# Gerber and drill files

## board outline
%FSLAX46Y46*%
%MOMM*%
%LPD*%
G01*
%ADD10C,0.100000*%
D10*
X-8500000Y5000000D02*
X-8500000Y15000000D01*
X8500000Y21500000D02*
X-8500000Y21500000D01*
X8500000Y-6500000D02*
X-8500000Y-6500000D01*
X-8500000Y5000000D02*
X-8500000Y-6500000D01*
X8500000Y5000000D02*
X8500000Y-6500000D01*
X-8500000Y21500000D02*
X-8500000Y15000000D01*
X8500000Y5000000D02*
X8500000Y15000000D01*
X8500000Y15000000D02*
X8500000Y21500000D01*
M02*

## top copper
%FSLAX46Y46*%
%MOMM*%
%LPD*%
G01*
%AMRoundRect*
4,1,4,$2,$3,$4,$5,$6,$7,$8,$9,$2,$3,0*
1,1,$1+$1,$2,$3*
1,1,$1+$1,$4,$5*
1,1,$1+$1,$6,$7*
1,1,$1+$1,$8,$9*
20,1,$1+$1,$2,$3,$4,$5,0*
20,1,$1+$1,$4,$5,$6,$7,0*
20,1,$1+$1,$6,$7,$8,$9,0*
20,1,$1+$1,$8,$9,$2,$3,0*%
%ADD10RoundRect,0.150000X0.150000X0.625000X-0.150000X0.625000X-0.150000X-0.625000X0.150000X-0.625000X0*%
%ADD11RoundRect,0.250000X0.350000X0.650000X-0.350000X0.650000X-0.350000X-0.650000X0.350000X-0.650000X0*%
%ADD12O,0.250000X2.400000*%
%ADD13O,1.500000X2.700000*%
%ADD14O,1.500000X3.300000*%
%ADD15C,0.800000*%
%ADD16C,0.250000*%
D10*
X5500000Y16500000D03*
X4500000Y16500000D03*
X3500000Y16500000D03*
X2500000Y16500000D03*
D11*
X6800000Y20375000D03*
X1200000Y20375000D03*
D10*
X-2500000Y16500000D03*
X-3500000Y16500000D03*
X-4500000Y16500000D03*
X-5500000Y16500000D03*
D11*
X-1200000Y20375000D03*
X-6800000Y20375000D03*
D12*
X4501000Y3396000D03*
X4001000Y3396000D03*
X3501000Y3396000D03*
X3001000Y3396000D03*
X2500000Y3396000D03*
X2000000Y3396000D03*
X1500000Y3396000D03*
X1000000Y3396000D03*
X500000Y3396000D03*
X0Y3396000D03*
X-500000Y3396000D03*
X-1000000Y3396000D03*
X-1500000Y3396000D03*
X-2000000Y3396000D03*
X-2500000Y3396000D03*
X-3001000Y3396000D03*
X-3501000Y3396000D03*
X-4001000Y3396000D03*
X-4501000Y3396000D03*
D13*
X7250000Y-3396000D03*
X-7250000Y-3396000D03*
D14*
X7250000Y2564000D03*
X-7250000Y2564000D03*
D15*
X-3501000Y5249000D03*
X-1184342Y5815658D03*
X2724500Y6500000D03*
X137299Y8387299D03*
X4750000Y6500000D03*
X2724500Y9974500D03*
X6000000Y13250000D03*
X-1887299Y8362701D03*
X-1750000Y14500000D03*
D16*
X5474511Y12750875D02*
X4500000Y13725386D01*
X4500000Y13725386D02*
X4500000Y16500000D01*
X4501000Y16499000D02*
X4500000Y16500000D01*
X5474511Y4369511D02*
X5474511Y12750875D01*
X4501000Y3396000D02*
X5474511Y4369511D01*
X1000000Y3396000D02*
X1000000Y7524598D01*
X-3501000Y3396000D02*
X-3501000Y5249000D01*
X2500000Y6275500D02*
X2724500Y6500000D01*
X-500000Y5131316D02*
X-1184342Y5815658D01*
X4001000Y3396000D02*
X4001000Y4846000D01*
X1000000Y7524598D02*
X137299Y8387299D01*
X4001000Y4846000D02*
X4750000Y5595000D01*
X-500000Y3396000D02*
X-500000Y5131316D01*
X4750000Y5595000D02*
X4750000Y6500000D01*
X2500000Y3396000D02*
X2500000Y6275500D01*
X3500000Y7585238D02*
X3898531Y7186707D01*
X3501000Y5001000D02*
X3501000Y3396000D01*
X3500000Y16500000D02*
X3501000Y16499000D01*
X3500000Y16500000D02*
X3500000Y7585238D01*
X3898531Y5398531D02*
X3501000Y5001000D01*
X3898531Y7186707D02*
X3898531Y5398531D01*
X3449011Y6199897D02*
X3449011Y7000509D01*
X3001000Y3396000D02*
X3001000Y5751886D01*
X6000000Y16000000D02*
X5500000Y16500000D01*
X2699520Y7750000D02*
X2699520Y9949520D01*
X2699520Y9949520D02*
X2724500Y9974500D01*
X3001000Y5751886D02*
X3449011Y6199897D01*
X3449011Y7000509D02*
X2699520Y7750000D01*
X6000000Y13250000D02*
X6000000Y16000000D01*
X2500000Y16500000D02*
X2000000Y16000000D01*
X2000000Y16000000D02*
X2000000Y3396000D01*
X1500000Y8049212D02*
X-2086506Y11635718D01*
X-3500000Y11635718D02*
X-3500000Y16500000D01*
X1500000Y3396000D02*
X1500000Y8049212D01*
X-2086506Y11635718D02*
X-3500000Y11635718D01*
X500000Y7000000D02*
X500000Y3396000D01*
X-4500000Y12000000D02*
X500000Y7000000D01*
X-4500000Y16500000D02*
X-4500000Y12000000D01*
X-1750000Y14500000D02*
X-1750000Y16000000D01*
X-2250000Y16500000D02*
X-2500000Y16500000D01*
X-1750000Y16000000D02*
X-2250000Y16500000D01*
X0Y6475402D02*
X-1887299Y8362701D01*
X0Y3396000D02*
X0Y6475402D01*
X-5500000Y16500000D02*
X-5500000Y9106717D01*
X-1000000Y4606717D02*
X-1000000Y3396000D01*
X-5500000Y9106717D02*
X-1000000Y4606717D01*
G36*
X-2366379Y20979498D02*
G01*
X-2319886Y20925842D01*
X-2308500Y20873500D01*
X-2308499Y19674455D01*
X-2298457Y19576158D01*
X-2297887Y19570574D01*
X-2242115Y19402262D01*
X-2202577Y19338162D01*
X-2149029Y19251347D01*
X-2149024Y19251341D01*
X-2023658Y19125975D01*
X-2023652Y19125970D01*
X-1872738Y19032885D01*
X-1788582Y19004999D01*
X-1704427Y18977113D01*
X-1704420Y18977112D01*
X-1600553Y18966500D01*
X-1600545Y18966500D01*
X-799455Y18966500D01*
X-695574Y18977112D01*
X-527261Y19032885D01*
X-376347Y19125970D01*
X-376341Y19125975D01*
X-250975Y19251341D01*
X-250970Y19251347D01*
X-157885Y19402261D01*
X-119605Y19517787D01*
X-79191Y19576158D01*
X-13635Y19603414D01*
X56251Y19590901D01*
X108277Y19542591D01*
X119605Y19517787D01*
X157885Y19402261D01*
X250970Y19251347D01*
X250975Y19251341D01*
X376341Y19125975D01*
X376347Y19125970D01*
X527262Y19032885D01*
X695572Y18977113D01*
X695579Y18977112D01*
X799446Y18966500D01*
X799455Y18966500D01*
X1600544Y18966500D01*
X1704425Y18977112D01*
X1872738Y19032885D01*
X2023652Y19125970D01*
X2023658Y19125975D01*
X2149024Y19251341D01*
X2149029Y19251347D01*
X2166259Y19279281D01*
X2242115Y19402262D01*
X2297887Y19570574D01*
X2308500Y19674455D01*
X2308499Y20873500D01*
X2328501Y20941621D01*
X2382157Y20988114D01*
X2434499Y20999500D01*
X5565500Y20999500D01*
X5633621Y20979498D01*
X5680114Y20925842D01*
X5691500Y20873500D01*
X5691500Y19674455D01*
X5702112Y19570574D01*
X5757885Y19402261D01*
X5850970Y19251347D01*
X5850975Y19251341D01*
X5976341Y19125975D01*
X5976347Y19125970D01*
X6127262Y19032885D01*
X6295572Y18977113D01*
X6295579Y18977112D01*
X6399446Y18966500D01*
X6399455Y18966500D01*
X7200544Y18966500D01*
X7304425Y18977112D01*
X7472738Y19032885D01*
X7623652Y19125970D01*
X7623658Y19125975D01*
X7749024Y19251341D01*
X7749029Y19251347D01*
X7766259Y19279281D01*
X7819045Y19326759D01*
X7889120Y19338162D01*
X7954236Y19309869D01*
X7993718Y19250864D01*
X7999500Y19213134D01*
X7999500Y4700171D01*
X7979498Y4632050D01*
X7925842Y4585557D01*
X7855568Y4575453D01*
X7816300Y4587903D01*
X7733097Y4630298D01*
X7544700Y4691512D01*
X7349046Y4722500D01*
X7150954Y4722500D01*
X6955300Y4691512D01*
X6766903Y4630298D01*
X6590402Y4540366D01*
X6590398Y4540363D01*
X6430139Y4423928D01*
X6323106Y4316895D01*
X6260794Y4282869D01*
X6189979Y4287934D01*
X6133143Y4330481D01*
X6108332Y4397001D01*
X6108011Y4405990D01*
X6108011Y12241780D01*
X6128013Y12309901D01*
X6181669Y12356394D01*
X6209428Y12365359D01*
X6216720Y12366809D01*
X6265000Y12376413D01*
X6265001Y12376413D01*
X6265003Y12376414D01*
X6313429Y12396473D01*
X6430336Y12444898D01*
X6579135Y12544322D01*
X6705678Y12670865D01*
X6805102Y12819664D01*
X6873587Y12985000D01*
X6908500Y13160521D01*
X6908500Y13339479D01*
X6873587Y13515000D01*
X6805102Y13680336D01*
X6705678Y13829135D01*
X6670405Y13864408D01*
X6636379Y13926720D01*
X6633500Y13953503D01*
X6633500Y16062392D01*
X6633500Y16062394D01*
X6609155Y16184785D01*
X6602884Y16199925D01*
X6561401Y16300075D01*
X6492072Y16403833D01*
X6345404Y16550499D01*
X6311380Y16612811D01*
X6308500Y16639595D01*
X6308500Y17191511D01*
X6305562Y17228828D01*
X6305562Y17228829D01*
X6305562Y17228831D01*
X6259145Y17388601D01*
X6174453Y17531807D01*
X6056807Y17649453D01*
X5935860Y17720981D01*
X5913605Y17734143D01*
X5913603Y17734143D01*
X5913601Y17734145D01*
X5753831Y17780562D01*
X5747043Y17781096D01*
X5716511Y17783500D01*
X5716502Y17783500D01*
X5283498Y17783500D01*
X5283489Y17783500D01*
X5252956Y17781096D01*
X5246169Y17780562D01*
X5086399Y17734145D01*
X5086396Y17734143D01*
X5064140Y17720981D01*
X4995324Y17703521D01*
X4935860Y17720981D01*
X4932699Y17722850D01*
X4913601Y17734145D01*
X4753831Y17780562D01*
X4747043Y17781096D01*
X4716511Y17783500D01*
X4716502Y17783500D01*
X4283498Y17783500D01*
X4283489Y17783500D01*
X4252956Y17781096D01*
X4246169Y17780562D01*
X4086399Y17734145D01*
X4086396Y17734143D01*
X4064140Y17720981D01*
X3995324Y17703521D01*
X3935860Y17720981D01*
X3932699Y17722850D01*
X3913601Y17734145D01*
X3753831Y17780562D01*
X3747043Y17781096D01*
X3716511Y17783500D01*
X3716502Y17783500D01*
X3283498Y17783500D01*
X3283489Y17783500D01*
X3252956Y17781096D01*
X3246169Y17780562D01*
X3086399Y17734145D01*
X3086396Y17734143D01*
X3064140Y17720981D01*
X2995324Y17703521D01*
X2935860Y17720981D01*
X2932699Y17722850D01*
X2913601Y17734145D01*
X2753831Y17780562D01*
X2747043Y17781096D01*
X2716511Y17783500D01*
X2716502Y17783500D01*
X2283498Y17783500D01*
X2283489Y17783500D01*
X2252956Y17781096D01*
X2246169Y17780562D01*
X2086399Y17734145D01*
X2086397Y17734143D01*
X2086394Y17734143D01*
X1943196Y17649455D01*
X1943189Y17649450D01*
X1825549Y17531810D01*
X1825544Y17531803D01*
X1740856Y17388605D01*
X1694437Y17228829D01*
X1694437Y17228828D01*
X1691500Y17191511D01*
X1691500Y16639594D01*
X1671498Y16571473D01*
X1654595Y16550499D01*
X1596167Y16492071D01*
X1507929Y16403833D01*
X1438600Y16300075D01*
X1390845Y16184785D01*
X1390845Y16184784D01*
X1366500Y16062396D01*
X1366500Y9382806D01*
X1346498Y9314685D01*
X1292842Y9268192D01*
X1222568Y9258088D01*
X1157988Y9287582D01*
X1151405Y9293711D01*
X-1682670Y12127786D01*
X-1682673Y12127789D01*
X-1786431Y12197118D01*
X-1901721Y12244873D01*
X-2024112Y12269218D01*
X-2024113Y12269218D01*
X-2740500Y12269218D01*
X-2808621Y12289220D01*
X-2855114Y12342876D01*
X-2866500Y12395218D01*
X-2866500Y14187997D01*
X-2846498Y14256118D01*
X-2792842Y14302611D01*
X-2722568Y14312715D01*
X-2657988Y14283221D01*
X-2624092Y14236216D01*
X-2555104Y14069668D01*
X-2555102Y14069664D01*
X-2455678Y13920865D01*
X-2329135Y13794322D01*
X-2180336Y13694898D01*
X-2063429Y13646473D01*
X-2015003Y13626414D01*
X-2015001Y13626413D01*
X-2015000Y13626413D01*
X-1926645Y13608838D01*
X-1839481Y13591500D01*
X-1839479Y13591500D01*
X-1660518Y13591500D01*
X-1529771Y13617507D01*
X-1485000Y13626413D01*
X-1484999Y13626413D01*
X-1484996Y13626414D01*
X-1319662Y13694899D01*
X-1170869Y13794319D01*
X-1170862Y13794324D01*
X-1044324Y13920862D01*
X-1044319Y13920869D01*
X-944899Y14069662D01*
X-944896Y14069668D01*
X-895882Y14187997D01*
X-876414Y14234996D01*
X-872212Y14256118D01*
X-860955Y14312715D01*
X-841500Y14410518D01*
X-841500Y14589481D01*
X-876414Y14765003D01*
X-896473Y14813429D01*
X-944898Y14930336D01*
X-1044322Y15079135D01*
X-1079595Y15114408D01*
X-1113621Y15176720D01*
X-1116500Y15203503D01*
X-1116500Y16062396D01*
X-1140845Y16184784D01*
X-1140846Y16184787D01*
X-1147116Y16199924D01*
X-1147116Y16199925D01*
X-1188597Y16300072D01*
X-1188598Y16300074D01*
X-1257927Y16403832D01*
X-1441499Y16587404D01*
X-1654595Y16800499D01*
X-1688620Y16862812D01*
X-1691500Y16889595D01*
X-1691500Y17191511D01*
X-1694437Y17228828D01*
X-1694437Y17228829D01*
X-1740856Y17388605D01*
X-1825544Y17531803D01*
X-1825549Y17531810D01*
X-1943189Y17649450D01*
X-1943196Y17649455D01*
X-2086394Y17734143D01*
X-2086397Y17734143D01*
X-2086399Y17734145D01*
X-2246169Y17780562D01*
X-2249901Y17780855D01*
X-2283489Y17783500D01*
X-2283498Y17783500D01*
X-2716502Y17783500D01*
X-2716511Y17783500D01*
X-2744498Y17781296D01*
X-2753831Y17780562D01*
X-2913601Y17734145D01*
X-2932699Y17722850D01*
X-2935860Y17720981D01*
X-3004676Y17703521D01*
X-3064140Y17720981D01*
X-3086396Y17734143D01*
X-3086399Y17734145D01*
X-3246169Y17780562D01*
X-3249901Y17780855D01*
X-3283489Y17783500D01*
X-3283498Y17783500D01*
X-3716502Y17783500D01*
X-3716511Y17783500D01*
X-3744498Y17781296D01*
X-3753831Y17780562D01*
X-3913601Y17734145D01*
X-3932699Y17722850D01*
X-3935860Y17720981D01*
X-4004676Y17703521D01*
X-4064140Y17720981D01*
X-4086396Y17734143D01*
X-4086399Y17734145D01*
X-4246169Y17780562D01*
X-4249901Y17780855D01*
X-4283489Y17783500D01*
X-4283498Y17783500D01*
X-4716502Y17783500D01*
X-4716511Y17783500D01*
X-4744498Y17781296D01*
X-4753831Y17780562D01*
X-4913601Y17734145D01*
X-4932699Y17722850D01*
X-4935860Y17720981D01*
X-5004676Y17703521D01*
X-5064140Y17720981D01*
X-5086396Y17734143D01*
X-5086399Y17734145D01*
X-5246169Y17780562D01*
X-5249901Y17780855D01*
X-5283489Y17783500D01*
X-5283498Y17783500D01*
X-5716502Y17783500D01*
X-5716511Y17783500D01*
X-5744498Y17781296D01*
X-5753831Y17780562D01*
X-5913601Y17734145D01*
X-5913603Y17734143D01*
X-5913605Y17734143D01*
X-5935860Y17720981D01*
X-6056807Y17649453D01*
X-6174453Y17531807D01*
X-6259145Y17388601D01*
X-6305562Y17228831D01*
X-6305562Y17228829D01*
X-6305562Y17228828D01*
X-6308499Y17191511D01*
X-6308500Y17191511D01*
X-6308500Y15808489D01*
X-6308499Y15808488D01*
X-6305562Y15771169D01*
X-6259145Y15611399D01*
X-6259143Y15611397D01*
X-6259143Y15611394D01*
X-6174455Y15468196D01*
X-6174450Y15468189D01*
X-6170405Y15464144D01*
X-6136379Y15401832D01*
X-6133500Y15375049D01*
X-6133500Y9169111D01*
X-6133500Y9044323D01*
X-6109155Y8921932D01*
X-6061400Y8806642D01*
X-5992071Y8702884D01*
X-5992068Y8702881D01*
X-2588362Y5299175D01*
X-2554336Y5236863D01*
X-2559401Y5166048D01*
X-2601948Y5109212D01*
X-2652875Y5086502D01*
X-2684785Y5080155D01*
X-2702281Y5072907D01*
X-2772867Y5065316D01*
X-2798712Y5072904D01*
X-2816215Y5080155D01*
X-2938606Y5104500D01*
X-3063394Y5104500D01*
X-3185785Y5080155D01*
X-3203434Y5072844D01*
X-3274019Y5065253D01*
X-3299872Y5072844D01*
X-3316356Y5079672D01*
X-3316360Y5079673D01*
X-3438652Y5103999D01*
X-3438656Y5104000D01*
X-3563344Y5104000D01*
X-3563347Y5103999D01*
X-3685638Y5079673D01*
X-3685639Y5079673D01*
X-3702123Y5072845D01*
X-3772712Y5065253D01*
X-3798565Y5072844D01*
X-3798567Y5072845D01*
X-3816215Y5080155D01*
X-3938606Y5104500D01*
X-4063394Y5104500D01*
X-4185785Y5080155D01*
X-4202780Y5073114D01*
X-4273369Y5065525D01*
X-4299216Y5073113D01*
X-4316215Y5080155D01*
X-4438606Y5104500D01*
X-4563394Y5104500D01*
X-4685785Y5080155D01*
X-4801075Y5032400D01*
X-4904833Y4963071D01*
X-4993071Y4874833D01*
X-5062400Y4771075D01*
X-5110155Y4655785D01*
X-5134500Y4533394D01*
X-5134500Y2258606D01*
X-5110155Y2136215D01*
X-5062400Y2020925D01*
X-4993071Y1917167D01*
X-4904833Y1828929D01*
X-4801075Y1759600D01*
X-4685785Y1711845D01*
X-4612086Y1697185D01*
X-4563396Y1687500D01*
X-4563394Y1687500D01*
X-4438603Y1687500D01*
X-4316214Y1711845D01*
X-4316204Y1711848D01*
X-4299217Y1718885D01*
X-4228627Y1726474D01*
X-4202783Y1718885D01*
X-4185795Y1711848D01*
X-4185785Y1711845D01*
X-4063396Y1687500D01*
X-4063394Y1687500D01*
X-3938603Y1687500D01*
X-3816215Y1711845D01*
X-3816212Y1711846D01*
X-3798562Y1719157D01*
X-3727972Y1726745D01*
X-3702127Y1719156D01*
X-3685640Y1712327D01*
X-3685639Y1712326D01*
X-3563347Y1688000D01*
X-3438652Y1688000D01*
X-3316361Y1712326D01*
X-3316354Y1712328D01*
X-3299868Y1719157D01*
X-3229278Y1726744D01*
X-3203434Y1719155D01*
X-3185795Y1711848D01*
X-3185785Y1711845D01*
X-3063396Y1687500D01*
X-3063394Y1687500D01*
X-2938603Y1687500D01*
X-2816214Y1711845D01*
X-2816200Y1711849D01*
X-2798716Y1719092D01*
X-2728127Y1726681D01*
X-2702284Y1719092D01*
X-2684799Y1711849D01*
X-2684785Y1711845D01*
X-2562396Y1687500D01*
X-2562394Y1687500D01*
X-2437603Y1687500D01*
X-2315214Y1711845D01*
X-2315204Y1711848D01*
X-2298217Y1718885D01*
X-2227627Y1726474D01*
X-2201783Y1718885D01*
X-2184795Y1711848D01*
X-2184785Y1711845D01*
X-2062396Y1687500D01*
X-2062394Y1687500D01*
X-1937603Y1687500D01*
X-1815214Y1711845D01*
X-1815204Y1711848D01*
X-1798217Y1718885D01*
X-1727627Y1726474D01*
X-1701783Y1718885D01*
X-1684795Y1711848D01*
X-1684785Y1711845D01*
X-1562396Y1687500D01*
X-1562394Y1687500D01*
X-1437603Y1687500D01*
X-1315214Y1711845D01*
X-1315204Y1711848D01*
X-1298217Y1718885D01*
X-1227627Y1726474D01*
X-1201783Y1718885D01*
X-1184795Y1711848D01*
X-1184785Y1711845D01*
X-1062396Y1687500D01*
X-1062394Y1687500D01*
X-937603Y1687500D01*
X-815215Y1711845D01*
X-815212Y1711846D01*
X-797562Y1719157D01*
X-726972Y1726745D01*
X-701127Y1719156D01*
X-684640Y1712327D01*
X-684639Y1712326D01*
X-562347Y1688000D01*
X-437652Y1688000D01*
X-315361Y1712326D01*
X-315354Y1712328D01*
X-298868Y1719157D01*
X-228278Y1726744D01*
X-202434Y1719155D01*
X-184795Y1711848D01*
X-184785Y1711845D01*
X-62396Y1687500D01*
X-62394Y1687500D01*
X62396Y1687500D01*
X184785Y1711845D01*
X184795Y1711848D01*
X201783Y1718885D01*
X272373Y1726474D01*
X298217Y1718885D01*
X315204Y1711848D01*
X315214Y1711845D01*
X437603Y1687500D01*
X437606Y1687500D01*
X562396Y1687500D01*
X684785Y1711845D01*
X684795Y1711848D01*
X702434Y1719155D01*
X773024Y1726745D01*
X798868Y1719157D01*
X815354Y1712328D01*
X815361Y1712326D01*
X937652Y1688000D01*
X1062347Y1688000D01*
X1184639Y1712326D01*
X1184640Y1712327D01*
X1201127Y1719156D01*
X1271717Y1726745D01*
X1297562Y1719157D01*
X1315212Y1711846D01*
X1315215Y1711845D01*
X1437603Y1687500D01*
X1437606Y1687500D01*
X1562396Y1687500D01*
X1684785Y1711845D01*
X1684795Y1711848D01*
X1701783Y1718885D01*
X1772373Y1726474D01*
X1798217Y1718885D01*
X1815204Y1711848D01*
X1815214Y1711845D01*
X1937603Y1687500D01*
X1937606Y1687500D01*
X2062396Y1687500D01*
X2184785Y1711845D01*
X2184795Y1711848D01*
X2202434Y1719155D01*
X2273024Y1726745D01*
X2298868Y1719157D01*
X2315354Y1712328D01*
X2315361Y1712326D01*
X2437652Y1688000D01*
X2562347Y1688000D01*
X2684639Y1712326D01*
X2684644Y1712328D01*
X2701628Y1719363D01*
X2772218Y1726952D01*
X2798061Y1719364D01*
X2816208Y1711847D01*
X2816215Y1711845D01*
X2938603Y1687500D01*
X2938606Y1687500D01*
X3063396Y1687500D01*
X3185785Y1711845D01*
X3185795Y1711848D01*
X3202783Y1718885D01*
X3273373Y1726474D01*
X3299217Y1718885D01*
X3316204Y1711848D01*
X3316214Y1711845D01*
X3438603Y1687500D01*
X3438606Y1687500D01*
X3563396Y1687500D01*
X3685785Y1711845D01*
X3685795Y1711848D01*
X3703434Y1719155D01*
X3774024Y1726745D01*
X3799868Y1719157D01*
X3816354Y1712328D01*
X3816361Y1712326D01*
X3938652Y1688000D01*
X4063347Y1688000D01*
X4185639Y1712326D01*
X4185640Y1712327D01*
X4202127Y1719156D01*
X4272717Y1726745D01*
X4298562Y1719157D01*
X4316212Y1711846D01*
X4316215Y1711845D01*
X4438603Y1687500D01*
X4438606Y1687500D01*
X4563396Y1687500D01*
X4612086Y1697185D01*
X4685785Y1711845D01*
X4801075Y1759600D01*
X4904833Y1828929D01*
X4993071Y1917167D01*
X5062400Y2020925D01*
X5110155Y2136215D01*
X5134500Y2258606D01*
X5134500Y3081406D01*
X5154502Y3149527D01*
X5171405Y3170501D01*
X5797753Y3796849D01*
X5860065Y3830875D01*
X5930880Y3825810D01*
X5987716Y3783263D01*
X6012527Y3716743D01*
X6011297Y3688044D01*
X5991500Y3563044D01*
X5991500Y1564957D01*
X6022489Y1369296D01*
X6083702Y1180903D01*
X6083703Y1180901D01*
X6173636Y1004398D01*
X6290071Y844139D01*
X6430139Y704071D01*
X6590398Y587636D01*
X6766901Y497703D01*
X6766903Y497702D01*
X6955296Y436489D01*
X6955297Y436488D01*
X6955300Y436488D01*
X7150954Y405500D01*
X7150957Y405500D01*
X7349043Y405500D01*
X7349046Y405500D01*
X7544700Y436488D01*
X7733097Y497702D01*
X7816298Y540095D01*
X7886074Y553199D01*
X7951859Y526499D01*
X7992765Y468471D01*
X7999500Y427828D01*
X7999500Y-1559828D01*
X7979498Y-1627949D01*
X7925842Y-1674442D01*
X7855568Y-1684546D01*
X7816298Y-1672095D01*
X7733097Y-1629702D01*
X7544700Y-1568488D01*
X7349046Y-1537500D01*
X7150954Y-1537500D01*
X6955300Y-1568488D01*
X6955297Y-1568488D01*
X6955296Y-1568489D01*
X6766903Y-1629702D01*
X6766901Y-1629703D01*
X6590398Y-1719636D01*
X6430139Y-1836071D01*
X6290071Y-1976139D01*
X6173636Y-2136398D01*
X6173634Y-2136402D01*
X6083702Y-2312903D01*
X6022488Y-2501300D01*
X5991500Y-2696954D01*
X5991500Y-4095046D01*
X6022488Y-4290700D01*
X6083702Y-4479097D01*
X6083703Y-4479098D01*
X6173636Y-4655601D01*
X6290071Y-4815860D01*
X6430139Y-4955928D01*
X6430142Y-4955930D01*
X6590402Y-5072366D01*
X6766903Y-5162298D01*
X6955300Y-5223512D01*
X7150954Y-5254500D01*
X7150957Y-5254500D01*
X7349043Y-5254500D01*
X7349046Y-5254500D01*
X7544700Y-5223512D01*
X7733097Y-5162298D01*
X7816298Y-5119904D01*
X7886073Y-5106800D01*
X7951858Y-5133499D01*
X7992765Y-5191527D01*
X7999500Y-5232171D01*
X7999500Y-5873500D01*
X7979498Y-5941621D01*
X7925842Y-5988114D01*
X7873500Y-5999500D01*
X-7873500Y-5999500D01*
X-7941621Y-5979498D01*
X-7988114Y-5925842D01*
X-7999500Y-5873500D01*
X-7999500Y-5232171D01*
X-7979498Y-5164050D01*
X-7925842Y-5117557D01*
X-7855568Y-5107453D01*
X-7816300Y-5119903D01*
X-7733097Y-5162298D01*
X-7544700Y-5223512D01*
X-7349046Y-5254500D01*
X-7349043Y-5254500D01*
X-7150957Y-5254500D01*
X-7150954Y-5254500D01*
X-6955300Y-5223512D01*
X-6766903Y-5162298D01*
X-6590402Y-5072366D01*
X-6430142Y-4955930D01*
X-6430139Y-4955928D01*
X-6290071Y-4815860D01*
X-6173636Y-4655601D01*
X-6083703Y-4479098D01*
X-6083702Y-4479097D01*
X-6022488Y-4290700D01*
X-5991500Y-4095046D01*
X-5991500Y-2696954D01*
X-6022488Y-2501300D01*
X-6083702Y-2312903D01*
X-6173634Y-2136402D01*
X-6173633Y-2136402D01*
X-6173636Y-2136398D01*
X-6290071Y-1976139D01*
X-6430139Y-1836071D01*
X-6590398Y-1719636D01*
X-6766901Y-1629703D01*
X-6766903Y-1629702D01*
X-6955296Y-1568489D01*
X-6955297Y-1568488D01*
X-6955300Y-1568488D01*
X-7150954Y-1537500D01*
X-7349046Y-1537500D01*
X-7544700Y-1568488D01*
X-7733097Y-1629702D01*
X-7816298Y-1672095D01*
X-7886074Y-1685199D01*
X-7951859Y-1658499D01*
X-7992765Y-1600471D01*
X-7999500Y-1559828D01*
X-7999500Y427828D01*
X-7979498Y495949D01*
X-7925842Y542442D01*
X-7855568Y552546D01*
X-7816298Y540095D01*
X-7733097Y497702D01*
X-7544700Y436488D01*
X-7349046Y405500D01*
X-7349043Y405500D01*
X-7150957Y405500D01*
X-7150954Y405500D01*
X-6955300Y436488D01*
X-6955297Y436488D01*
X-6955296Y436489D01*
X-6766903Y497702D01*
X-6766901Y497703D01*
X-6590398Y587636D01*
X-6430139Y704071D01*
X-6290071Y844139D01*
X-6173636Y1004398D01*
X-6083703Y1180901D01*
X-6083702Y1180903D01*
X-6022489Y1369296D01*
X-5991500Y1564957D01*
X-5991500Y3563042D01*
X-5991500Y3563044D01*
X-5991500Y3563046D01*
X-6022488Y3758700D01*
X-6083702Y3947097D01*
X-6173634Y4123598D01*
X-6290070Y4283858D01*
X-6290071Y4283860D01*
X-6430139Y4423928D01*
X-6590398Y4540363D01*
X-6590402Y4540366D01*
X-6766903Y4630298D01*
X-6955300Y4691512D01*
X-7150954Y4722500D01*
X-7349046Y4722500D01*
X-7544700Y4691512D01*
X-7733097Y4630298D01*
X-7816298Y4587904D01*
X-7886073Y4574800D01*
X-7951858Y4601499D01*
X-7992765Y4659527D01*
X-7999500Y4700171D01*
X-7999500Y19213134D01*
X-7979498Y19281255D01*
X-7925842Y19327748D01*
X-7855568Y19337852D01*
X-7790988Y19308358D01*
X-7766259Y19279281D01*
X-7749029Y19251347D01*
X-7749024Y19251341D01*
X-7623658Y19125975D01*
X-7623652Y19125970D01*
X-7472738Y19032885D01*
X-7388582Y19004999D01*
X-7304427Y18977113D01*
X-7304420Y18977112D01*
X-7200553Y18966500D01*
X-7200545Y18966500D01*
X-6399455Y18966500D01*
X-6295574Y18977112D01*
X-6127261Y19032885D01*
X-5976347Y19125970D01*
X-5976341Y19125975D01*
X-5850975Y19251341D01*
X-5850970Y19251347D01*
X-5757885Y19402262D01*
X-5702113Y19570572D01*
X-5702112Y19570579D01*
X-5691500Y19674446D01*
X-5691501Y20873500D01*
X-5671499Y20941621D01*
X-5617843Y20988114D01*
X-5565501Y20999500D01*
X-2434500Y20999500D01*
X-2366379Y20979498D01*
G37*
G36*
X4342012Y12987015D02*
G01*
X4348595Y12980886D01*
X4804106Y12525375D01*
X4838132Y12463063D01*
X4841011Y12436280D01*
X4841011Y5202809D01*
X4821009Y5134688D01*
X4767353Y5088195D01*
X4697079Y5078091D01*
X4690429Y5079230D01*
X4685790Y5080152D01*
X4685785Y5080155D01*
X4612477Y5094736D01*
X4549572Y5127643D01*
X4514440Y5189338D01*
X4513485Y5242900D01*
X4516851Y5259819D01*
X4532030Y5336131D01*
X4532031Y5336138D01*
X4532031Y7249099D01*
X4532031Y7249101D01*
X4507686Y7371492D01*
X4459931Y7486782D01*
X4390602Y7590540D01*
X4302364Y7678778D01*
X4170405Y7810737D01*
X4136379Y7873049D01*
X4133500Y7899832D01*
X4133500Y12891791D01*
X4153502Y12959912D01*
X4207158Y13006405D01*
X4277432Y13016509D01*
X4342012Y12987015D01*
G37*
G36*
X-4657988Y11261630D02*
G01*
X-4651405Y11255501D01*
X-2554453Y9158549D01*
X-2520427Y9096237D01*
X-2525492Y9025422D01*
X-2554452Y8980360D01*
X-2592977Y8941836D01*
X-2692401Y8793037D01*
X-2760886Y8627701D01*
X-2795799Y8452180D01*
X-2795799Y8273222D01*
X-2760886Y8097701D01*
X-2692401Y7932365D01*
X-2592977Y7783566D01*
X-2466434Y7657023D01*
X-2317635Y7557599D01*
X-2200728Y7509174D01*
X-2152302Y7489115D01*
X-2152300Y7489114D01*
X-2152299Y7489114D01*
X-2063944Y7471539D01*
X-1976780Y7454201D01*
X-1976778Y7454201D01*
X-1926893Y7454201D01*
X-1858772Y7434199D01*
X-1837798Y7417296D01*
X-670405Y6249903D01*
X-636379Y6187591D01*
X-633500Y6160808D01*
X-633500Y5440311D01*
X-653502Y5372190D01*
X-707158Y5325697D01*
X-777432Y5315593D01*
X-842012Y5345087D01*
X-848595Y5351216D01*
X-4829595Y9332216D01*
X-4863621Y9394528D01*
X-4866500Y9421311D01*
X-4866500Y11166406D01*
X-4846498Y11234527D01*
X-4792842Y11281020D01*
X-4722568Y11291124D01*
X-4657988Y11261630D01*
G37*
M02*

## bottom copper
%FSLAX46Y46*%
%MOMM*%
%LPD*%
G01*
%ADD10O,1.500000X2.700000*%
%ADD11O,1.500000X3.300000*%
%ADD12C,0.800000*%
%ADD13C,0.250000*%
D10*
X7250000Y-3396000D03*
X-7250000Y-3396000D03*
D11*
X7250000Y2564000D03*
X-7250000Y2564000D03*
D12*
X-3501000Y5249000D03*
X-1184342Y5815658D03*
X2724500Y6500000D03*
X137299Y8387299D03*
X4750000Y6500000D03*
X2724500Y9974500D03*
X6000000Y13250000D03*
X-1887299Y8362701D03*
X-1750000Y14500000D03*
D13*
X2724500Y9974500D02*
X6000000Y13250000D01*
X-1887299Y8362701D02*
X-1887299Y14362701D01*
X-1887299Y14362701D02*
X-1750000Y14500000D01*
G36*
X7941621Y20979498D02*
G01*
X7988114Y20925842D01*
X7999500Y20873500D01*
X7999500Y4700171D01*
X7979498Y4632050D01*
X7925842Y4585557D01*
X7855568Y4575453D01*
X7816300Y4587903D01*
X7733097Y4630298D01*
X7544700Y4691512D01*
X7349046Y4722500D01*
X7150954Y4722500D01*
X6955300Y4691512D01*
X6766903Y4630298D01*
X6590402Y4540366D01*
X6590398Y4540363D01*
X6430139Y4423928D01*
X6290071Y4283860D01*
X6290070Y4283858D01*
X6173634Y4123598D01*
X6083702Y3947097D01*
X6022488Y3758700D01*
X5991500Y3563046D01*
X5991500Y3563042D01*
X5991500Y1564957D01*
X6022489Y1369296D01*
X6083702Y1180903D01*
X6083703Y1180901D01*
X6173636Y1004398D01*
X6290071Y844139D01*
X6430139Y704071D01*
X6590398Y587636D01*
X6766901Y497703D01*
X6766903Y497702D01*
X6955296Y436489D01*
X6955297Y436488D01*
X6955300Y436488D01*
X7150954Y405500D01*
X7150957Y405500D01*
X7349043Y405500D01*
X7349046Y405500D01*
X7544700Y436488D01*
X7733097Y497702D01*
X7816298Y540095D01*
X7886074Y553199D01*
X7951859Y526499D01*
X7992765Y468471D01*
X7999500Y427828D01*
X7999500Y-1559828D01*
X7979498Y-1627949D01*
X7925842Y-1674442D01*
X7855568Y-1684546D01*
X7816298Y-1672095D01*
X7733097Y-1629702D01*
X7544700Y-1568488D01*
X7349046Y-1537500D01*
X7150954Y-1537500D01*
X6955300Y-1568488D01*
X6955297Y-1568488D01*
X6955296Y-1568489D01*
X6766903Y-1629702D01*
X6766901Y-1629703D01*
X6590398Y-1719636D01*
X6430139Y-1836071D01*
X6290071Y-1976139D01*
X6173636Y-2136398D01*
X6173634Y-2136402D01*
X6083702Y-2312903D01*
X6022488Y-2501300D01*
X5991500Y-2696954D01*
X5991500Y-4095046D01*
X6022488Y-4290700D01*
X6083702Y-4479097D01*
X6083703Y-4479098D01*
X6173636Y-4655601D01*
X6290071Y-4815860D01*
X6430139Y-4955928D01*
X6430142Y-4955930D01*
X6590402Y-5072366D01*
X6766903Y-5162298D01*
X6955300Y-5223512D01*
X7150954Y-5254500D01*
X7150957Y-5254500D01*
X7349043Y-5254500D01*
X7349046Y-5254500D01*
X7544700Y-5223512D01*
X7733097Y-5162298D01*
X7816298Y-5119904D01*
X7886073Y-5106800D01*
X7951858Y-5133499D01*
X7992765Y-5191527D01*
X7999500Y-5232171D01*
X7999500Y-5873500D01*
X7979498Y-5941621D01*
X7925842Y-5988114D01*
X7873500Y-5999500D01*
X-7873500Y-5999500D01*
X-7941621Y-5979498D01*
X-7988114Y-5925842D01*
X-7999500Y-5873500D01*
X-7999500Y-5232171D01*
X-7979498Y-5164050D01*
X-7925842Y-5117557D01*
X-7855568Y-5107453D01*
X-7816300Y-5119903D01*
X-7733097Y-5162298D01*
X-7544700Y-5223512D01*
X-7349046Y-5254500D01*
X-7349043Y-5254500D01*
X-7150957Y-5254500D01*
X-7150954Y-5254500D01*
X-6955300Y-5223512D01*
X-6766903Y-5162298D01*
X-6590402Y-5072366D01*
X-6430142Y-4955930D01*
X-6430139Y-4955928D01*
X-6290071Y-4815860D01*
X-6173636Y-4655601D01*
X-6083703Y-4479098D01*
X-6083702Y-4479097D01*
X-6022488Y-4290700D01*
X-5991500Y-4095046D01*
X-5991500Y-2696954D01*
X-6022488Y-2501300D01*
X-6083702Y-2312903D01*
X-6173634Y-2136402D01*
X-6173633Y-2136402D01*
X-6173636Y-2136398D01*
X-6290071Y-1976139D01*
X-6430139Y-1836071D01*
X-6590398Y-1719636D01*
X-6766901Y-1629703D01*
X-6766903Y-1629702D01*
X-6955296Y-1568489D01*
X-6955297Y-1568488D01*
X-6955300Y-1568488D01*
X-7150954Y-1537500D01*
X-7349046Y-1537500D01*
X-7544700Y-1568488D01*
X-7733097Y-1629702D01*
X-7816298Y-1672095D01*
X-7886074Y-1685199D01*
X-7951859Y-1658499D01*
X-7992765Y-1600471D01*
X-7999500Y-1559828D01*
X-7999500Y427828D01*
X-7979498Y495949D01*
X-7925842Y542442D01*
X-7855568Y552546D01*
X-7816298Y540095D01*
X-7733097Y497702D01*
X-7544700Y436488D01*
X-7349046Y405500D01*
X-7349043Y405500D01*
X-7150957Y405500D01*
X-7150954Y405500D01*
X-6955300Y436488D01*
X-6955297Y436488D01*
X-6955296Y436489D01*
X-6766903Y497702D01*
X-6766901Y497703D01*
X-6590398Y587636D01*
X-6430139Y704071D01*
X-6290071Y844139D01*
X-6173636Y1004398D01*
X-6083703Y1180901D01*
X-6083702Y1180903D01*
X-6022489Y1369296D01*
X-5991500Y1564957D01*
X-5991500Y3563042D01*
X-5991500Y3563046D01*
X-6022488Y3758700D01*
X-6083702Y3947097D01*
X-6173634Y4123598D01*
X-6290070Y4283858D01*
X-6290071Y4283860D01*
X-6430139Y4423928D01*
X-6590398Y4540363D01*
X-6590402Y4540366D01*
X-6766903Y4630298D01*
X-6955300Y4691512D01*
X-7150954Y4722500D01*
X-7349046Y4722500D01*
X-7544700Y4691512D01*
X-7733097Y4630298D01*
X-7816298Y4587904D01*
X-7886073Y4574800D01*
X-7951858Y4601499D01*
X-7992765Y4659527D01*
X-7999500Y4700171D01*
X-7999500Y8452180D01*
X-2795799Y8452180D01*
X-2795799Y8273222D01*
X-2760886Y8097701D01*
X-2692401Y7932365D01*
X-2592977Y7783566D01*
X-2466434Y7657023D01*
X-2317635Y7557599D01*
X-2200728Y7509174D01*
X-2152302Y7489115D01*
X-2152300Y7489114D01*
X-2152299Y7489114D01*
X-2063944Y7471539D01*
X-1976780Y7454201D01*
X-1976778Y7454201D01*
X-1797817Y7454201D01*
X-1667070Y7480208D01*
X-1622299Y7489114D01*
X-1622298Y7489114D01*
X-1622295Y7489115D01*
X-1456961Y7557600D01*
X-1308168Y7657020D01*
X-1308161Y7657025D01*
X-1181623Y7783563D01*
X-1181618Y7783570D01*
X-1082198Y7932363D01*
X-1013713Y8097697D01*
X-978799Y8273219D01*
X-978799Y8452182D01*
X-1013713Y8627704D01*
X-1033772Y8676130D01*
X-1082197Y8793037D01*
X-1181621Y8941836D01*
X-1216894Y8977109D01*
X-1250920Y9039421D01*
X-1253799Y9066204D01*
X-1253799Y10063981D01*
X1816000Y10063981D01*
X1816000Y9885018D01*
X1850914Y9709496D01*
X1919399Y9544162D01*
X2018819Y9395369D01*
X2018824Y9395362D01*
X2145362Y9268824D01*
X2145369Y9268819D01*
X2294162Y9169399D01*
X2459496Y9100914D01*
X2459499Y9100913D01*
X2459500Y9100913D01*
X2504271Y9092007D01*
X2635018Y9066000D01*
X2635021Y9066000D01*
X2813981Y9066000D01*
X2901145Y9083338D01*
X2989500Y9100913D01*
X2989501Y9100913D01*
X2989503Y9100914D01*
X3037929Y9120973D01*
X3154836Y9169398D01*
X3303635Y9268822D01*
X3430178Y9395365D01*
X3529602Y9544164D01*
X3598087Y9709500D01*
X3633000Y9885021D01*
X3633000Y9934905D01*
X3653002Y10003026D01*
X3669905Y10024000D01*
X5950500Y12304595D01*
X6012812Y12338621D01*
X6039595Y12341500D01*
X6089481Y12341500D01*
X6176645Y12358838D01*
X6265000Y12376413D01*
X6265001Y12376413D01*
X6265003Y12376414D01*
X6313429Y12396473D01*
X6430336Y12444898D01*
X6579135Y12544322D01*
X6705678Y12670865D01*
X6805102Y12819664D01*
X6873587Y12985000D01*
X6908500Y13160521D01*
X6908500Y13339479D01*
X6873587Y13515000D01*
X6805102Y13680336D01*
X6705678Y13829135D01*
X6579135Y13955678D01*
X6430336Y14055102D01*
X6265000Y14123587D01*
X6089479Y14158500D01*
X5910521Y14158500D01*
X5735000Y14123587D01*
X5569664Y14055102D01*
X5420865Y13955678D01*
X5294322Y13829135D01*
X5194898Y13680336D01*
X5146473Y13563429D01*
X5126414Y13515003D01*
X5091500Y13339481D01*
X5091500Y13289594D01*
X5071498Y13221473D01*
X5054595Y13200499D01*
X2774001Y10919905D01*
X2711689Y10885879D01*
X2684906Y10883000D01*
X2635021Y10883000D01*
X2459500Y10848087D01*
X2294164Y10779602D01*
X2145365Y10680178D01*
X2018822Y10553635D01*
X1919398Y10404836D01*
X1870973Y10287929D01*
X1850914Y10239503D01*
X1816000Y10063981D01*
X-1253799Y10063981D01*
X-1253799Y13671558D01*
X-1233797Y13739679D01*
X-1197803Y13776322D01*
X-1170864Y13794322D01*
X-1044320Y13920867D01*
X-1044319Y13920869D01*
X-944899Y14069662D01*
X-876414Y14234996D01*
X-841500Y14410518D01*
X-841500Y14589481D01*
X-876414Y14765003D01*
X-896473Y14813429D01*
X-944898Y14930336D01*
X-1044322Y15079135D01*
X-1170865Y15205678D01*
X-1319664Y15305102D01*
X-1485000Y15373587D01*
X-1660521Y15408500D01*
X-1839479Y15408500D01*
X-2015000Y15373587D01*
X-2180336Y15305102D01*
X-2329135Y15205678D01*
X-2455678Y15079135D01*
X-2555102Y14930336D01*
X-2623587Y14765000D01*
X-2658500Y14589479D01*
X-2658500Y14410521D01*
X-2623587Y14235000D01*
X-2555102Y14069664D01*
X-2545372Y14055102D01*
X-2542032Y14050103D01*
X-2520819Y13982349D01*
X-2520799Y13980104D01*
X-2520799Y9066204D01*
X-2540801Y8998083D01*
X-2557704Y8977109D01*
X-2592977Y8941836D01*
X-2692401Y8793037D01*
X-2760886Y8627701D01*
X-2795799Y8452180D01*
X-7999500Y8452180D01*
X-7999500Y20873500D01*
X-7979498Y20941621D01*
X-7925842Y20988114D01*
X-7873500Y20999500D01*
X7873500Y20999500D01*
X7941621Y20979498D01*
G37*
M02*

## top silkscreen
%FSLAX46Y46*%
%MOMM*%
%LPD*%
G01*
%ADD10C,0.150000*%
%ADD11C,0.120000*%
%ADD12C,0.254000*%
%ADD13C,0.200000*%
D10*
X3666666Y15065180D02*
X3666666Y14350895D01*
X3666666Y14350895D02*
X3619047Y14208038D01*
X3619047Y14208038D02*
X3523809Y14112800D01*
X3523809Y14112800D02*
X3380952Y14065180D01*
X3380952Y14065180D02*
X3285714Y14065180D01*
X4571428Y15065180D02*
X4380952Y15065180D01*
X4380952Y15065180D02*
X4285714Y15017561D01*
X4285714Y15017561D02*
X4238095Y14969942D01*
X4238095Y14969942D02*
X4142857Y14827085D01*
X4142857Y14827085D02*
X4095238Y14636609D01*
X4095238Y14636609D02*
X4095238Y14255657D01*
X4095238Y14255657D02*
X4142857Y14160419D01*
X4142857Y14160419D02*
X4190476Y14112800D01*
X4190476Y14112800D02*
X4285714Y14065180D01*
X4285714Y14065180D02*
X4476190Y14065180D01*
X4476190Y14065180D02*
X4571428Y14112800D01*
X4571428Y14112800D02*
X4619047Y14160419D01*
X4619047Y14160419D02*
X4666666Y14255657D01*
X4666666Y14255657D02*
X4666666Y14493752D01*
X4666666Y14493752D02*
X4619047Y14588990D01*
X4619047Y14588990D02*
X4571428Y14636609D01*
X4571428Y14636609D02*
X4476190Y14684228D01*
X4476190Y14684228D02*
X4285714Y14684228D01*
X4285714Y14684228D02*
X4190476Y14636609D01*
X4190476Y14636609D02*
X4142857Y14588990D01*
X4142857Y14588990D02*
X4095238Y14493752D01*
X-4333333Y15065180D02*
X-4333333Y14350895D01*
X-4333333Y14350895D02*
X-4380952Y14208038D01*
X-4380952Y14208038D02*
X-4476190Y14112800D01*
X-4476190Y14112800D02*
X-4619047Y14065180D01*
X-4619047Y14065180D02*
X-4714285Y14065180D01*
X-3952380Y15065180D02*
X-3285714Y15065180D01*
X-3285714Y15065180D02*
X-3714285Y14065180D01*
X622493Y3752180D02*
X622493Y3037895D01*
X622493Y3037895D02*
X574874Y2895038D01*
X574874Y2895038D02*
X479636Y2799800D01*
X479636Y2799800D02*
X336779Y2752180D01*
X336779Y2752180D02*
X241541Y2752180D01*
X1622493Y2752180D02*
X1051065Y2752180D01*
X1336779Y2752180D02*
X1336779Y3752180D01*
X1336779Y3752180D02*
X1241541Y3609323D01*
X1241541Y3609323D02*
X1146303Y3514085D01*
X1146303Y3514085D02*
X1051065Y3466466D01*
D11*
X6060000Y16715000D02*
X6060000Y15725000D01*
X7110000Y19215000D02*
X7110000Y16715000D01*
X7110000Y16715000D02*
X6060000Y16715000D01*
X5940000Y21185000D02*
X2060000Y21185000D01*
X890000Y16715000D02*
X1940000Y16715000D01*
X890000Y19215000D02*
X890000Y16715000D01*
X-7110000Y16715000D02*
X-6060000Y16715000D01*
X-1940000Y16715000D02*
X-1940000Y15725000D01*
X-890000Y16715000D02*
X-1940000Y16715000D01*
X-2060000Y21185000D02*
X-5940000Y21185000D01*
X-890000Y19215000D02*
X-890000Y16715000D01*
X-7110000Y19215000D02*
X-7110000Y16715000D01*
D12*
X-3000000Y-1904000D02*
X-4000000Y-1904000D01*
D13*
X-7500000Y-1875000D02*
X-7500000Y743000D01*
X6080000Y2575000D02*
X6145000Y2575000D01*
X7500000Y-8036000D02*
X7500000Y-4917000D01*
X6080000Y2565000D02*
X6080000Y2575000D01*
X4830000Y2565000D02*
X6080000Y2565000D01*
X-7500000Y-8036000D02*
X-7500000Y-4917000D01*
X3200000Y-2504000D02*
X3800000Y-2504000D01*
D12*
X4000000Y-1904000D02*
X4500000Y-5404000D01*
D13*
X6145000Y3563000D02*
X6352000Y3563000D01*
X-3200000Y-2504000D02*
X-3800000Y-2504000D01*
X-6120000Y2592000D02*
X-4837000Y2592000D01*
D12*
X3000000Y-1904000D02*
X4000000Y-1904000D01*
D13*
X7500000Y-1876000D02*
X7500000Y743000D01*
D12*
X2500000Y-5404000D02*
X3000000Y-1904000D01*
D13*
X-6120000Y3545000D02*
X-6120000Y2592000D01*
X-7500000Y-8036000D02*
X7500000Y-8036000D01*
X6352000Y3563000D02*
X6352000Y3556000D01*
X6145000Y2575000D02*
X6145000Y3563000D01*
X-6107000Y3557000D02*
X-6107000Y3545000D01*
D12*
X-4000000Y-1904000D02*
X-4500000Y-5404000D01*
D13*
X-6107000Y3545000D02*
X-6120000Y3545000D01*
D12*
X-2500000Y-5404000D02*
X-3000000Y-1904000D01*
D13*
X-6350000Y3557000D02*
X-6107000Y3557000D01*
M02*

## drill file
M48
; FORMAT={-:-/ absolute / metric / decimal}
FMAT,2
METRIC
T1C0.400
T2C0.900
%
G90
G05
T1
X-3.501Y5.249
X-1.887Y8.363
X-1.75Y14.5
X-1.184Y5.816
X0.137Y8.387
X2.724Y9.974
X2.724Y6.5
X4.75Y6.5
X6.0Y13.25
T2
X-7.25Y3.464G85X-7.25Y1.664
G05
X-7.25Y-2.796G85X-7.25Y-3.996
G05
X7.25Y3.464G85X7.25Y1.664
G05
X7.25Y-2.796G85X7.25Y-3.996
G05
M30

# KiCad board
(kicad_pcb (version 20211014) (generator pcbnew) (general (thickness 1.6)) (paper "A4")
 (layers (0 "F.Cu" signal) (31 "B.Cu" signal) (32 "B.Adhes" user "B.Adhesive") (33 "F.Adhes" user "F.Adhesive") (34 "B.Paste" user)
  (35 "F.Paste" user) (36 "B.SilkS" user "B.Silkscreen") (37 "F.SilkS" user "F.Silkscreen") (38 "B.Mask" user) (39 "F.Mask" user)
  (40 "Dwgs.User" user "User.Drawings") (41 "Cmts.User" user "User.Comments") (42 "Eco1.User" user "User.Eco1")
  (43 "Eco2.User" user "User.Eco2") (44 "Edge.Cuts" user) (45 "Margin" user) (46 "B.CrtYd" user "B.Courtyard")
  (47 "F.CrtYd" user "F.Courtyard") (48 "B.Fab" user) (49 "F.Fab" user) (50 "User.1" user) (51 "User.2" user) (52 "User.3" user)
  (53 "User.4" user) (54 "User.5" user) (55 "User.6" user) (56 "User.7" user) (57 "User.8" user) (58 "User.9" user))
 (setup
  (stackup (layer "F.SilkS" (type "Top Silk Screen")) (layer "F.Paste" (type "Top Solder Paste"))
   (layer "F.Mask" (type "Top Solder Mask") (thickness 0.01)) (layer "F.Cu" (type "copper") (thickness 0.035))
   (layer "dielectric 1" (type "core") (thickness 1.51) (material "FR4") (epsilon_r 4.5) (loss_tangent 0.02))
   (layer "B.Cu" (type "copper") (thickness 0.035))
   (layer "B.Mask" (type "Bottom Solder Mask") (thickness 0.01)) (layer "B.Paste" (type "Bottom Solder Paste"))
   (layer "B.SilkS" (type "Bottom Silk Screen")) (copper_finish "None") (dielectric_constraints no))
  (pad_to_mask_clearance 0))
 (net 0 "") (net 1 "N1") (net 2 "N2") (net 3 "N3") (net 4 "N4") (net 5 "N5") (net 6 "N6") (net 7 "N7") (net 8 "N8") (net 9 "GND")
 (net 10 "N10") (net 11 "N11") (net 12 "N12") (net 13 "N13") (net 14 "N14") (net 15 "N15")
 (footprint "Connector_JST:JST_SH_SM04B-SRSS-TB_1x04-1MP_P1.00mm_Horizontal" (layer "F.Cu") (at 4 -18.5 180)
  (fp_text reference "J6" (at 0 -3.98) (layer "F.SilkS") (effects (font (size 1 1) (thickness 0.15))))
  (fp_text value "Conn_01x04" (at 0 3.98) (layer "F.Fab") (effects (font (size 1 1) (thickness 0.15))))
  (fp_line (start -2.06 -1.785) (end -2.06 -2.775) (layer "F.SilkS") (width 0.12))
  (fp_line (start -3.11 0.715) (end -3.11 -1.785) (layer "F.SilkS") (width 0.12))
  (fp_line (start -3.11 -1.785) (end -2.06 -1.785) (layer "F.SilkS") (width 0.12))
  (fp_line (start -1.94 2.685) (end 1.94 2.685) (layer "F.SilkS") (width 0.12))
  (fp_line (start 3.11 -1.785) (end 2.06 -1.785) (layer "F.SilkS") (width 0.12))
  (fp_line (start 3.11 0.715) (end 3.11 -1.785) (layer "F.SilkS") (width 0.12))
  (pad "1" smd roundrect (at -1.5 -2 180) (size 0.6 1.55) (layers "F.Cu" "F.Paste" "F.Mask") (roundrect_rratio 0.25) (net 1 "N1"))
  (pad "2" smd roundrect (at -0.5 -2 180) (size 0.6 1.55) (layers "F.Cu" "F.Paste" "F.Mask") (roundrect_rratio 0.25) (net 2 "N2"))
  (pad "3" smd roundrect (at 0.5 -2 180) (size 0.6 1.55) (layers "F.Cu" "F.Paste" "F.Mask") (roundrect_rratio 0.25) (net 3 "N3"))
  (pad "4" smd roundrect (at 1.5 -2 180) (size 0.6 1.55) (layers "F.Cu" "F.Paste" "F.Mask") (roundrect_rratio 0.25) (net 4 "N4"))
  (pad "MP" smd roundrect (at -2.8 1.875 180) (size 1.2 1.8) (layers "F.Cu" "F.Paste" "F.Mask") (roundrect_rratio 0.2083333333))
  (pad "MP" smd roundrect (at 2.8 1.875 180) (size 1.2 1.8) (layers "F.Cu" "F.Paste" "F.Mask") (roundrect_rratio 0.2083333333)))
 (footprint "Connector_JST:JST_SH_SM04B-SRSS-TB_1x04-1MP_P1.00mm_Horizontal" (layer "F.Cu") (at -4 -18.5 180)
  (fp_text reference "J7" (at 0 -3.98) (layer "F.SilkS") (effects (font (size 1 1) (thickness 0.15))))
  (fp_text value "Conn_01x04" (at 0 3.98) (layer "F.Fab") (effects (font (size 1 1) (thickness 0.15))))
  (fp_line (start 3.11 -1.785) (end 2.06 -1.785) (layer "F.SilkS") (width 0.12))
  (fp_line (start -2.06 -1.785) (end -2.06 -2.775) (layer "F.SilkS") (width 0.12))
  (fp_line (start -3.11 -1.785) (end -2.06 -1.785) (layer "F.SilkS") (width 0.12))
  (fp_line (start -1.94 2.685) (end 1.94 2.685) (layer "F.SilkS") (width 0.12))
  (fp_line (start -3.11 0.715) (end -3.11 -1.785) (layer "F.SilkS") (width 0.12))
  (fp_line (start 3.11 0.715) (end 3.11 -1.785) (layer "F.SilkS") (width 0.12))
  (pad "1" smd roundrect (at -1.5 -2 180) (size 0.6 1.55) (layers "F.Cu" "F.Paste" "F.Mask") (roundrect_rratio 0.25) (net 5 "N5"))
  (pad "2" smd roundrect (at -0.5 -2 180) (size 0.6 1.55) (layers "F.Cu" "F.Paste" "F.Mask") (roundrect_rratio 0.25) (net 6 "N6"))
  (pad "3" smd roundrect (at 0.5 -2 180) (size 0.6 1.55) (layers "F.Cu" "F.Paste" "F.Mask") (roundrect_rratio 0.25) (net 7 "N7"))
  (pad "4" smd roundrect (at 1.5 -2 180) (size 0.6 1.55) (layers "F.Cu" "F.Paste" "F.Mask") (roundrect_rratio 0.25) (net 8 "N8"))
  (pad "MP" smd roundrect (at -2.8 1.875 180) (size 1.2 1.8) (layers "F.Cu" "F.Paste" "F.Mask") (roundrect_rratio 0.2083333333))
  (pad "MP" smd roundrect (at 2.8 1.875 180) (size 1.2 1.8) (layers "F.Cu" "F.Paste" "F.Mask") (roundrect_rratio 0.2083333333)))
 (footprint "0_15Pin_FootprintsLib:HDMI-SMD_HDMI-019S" (layer "F.Cu") (at 0 0)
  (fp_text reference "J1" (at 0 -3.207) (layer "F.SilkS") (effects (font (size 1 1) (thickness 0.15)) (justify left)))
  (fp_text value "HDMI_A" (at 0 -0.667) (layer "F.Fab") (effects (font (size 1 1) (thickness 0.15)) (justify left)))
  (fp_line (start -3 1.904) (end -4 1.904) (layer "F.SilkS") (width 0.254))
  (fp_line (start -7.5 1.875) (end -7.5 -0.743) (layer "F.SilkS") (width 0.2))
  (fp_line (start 6.08 -2.575) (end 6.145 -2.575) (layer "F.SilkS") (width 0.2))
  (fp_line (start 7.5 8.036) (end 7.5 4.917) (layer "F.SilkS") (width 0.2))
  (fp_line (start 6.08 -2.565) (end 6.08 -2.575) (layer "F.SilkS") (width 0.2))
  (fp_line (start 4.83 -2.565) (end 6.08 -2.565) (layer "F.SilkS") (width 0.2))
  (fp_line (start -7.5 8.036) (end -7.5 4.917) (layer "F.SilkS") (width 0.2))
  (fp_line (start 3.2 2.504) (end 3.8 2.504) (layer "F.SilkS") (width 0.2))
  (fp_line (start 4 1.904) (end 4.5 5.404) (layer "F.SilkS") (width 0.254))
  (fp_line (start 6.145 -3.563) (end 6.352 -3.563) (layer "F.SilkS") (width 0.2))
  (fp_line (start -3.2 2.504) (end -3.8 2.504) (layer "F.SilkS") (width 0.2))
  (fp_line (start -6.12 -2.592) (end -4.837 -2.592) (layer "F.SilkS") (width 0.2))
  (fp_line (start 3 1.904) (end 4 1.904) (layer "F.SilkS") (width 0.254))
  (fp_line (start 7.5 1.876) (end 7.5 -0.743) (layer "F.SilkS") (width 0.2))
  (fp_line (start 2.5 5.404) (end 3 1.904) (layer "F.SilkS") (width 0.254))
  (fp_line (start -6.12 -3.545) (end -6.12 -2.592) (layer "F.SilkS") (width 0.2))
  (fp_line (start -7.5 8.036) (end 7.5 8.036) (layer "F.SilkS") (width 0.2))
  (fp_line (start 6.352 -3.563) (end 6.352 -3.556) (layer "F.SilkS") (width 0.2))
  (fp_line (start 6.145 -2.575) (end 6.145 -3.563) (layer "F.SilkS") (width 0.2))
  (fp_line (start -6.107 -3.557) (end -6.107 -3.545) (layer "F.SilkS") (width 0.2))
  (fp_line (start -4 1.904) (end -4.5 5.404) (layer "F.SilkS") (width 0.254))
  (fp_line (start -6.107 -3.545) (end -6.12 -3.545) (layer "F.SilkS") (width 0.2))
  (fp_line (start -2.5 5.404) (end -3 1.904) (layer "F.SilkS") (width 0.254))
  (fp_line (start -6.35 -3.557) (end -6.107 -3.557) (layer "F.SilkS") (width 0.2))
  (pad "1" smd oval (at 4.501 -3.396) (size 0.25 2.4) (layers "F.Cu" "F.Paste" "F.Mask") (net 2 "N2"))
  (pad "2" smd oval (at 4.001 -3.396) (size 0.25 2.4) (layers "F.Cu" "F.Paste" "F.Mask") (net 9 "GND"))
  (pad "3" smd oval (at 3.501 -3.396) (size 0.25 2.4) (layers "F.Cu" "F.Paste" "F.Mask") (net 3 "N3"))
  (pad "4" smd oval (at 3.001 -3.396) (size 0.25 2.4) (layers "F.Cu" "F.Paste" "F.Mask") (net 1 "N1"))
  (pad "5" smd oval (at 2.5 -3.396) (size 0.25 2.4) (layers "F.Cu" "F.Paste" "F.Mask") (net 9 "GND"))
  (pad "6" smd oval (at 2 -3.396) (size 0.25 2.4) (layers "F.Cu" "F.Paste" "F.Mask") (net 4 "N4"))
  (pad "7" smd oval (at 1.5 -3.396) (size 0.25 2.4) (layers "F.Cu" "F.Paste" "F.Mask") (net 6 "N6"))
  (pad "8" smd oval (at 1 -3.396) (size 0.25 2.4) (layers "F.Cu" "F.Paste" "F.Mask") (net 9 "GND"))
  (pad "9" smd oval (at 0.5 -3.396) (size 0.25 2.4) (layers "F.Cu" "F.Paste" "F.Mask") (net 7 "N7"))
  (pad "10" smd oval (at 0 -3.396) (size 0.25 2.4) (layers "F.Cu" "F.Paste" "F.Mask") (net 5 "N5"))
  (pad "11" smd oval (at -0.5 -3.396) (size 0.25 2.4) (layers "F.Cu" "F.Paste" "F.Mask") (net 9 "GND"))
  (pad "12" smd oval (at -1 -3.396) (size 0.25 2.4) (layers "F.Cu" "F.Paste" "F.Mask") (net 8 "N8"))
  (pad "13" smd oval (at -1.5 -3.396) (size 0.25 2.4) (layers "F.Cu" "F.Paste" "F.Mask") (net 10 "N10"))
  (pad "14" smd oval (at -2 -3.396) (size 0.25 2.4) (layers "F.Cu" "F.Paste" "F.Mask") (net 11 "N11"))
  (pad "15" smd oval (at -2.5 -3.396) (size 0.25 2.4) (layers "F.Cu" "F.Paste" "F.Mask") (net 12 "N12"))
  (pad "16" smd oval (at -3.001 -3.396) (size 0.25 2.4) (layers "F.Cu" "F.Paste" "F.Mask") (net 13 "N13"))
  (pad "17" smd oval (at -3.501 -3.396) (size 0.25 2.4) (layers "F.Cu" "F.Paste" "F.Mask") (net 9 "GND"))
  (pad "18" smd oval (at -4.001 -3.396) (size 0.25 2.4) (layers "F.Cu" "F.Paste" "F.Mask") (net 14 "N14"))
  (pad "19" smd oval (at -4.501 -3.396) (size 0.25 2.4) (layers "F.Cu" "F.Paste" "F.Mask") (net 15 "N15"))
  (pad "20" thru_hole oval (at 7.25 3.396) (size 1.5 2.7) (drill oval 0.9 2.1) (layers *.Cu *.Mask))
  (pad "21" thru_hole oval (at -7.25 3.396) (size 1.5 2.7) (drill oval 0.9 2.1) (layers *.Cu *.Mask))
  (pad "22" thru_hole oval (at 7.25 -2.564) (size 1.5 3.3) (drill oval 0.9 2.7) (layers *.Cu *.Mask))
  (pad "23" thru_hole oval (at -7.25 -2.564) (size 1.5 3.3) (drill oval 0.9 2.7) (layers *.Cu *.Mask)))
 (gr_line (start -8.5 -5) (end -8.5 -15) (layer "Edge.Cuts") (width 0.1))
 (gr_line (start 8.5 -21.5) (end -8.5 -21.5) (layer "Edge.Cuts") (width 0.1))
 (gr_line (start 8.5 6.5) (end -8.5 6.5) (layer "Edge.Cuts") (width 0.1))
 (gr_line (start -8.5 -5) (end -8.5 6.5) (layer "Edge.Cuts") (width 0.1))
 (gr_line (start 8.5 -5) (end 8.5 6.5) (layer "Edge.Cuts") (width 0.1))
 (gr_line (start -8.5 -21.5) (end -8.5 -15) (layer "Edge.Cuts") (width 0.1))
 (gr_line (start 8.5 -5) (end 8.5 -15) (layer "Edge.Cuts") (width 0.1))
 (gr_line (start 8.5 -15) (end 8.5 -21.5) (layer "Edge.Cuts") (width 0.1))
 (segment (start 5.474511 -12.750875) (end 4.5 -13.725386) (width 0.25) (layer "F.Cu") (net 2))
 (segment (start 4.5 -13.725386) (end 4.5 -16.5) (width 0.25) (layer "F.Cu") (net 2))
 (segment (start 4.501 -16.499) (end 4.5 -16.5) (width 0.25) (layer "F.Cu") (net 2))
 (segment (start 5.474511 -4.369511) (end 5.474511 -12.750875) (width 0.25) (layer "F.Cu") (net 2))
 (segment (start 4.501 -3.396) (end 5.474511 -4.369511) (width 0.25) (layer "F.Cu") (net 2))
 (segment (start 1 -3.396) (end 1 -7.524598) (width 0.25) (layer "F.Cu") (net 9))
 (segment (start -3.501 -3.396) (end -3.501 -5.249) (width 0.25) (layer "F.Cu") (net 9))
 (segment (start 2.5 -6.2755) (end 2.7245 -6.5) (width 0.25) (layer "F.Cu") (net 9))
 (segment (start -0.5 -5.131316) (end -1.184342 -5.815658) (width 0.25) (layer "F.Cu") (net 9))
 (segment (start 4.001 -3.396) (end 4.001 -4.846) (width 0.25) (layer "F.Cu") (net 9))
 (segment (start 1 -7.524598) (end 0.137299 -8.387299) (width 0.25) (layer "F.Cu") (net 9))
 (segment (start 4.001 -4.846) (end 4.75 -5.595) (width 0.25) (layer "F.Cu") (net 9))
 (segment (start -0.5 -3.396) (end -0.5 -5.131316) (width 0.25) (layer "F.Cu") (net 9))
 (segment (start 4.75 -5.595) (end 4.75 -6.5) (width 0.25) (layer "F.Cu") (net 9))
 (segment (start 2.5 -3.396) (end 2.5 -6.2755) (width 0.25) (layer "F.Cu") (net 9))
 (via (at -3.501 -5.249) (size 0.8) (drill 0.4) (layers "F.Cu" "B.Cu") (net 9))
 (via (at -1.184342 -5.815658) (size 0.8) (drill 0.4) (layers "F.Cu" "B.Cu") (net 9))
 (via (at 2.7245 -6.5) (size 0.8) (drill 0.4) (layers "F.Cu" "B.Cu") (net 9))
 (via (at 0.137299 -8.387299) (size 0.8) (drill 0.4) (layers "F.Cu" "B.Cu") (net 9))
 (via (at 4.75 -6.5) (size 0.8) (drill 0.4) (layers "F.Cu" "B.Cu") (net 9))
 (segment (start 3.5 -7.585238) (end 3.898531 -7.186707) (width 0.25) (layer "F.Cu") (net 3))
 (segment (start 3.501 -5.001) (end 3.501 -3.396) (width 0.25) (layer "F.Cu") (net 3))
 (segment (start 3.5 -16.5) (end 3.501 -16.499) (width 0.25) (layer "F.Cu") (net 3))
 (segment (start 3.5 -16.5) (end 3.5 -7.585238) (width 0.25) (layer "F.Cu") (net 3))
 (segment (start 3.898531 -5.398531) (end 3.501 -5.001) (width 0.25) (layer "F.Cu") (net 3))
 (segment (start 3.898531 -7.186707) (end 3.898531 -5.398531) (width 0.25) (layer "F.Cu") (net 3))
 (segment (start 3.449011 -6.199897) (end 3.449011 -7.000509) (width 0.25) (layer "F.Cu") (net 1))
 (segment (start 3.001 -3.396) (end 3.001 -5.751886) (width 0.25) (layer "F.Cu") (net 1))
 (segment (start 6 -16) (end 5.5 -16.5) (width 0.25) (layer "F.Cu") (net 1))
 (segment (start 2.69952 -7.75) (end 2.69952 -9.94952) (width 0.25) (layer "F.Cu") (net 1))
 (segment (start 2.69952 -9.94952) (end 2.7245 -9.9745) (width 0.25) (layer "F.Cu") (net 1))
 (segment (start 3.001 -5.751886) (end 3.449011 -6.199897) (width 0.25) (layer "F.Cu") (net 1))
 (segment (start 3.449011 -7.000509) (end 2.69952 -7.75) (width 0.25) (layer "F.Cu") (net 1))
 (segment (start 6 -13.25) (end 6 -16) (width 0.25) (layer "F.Cu") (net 1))
 (via (at 2.7245 -9.9745) (size 0.8) (drill 0.4) (layers "F.Cu" "B.Cu") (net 1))
 (via (at 6 -13.25) (size 0.8) (drill 0.4) (layers "F.Cu" "B.Cu") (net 1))
 (segment (start 2.7245 -9.9745) (end 6 -13.25) (width 0.25) (layer "B.Cu") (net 1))
 (segment (start 2.5 -16.5) (end 2 -16) (width 0.25) (layer "F.Cu") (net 4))
 (segment (start 2 -16) (end 2 -3.396) (width 0.25) (layer "F.Cu") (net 4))
 (segment (start 1.5 -8.049212) (end -2.086506 -11.635718) (width 0.25) (layer "F.Cu") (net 6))
 (segment (start -3.5 -11.635718) (end -3.5 -16.5) (width 0.25) (layer "F.Cu") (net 6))
 (segment (start 1.5 -3.396) (end 1.5 -8.049212) (width 0.25) (layer "F.Cu") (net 6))
 (segment (start -2.086506 -11.635718) (end -3.5 -11.635718) (width 0.25) (layer "F.Cu") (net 6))
 (segment (start 0.5 -7) (end 0.5 -3.396) (width 0.25) (layer "F.Cu") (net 7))
 (segment (start -4.5 -12) (end 0.5 -7) (width 0.25) (layer "F.Cu") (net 7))
 (segment (start -4.5 -16.5) (end -4.5 -12) (width 0.25) (layer "F.Cu") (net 7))
 (segment (start -1.75 -14.5) (end -1.75 -16) (width 0.25) (layer "F.Cu") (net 5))
 (segment (start -2.25 -16.5) (end -2.5 -16.5) (width 0.25) (layer "F.Cu") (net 5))
 (segment (start -1.75 -16) (end -2.25 -16.5) (width 0.25) (layer "F.Cu") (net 5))
 (segment (start 0 -6.475402) (end -1.887299 -8.362701) (width 0.25) (layer "F.Cu") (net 5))
 (segment (start 0 -3.396) (end 0 -6.475402) (width 0.25) (layer "F.Cu") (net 5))
 (via (at -1.887299 -8.362701) (size 0.8) (drill 0.4) (layers "F.Cu" "B.Cu") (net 5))
 (via (at -1.75 -14.5) (size 0.8) (drill 0.4) (layers "F.Cu" "B.Cu") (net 5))
 (segment (start -1.887299 -8.362701) (end -1.887299 -14.362701) (width 0.25) (layer "B.Cu") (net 5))
 (segment (start -1.887299 -14.362701) (end -1.75 -14.5) (width 0.25) (layer "B.Cu") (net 5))
 (segment (start -5.5 -16.5) (end -5.5 -9.106717) (width 0.25) (layer "F.Cu") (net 8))
 (segment (start -1 -4.606717) (end -1 -3.396) (width 0.25) (layer "F.Cu") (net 8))
 (segment (start -5.5 -9.106717) (end -1 -4.606717) (width 0.25) (layer "F.Cu") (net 8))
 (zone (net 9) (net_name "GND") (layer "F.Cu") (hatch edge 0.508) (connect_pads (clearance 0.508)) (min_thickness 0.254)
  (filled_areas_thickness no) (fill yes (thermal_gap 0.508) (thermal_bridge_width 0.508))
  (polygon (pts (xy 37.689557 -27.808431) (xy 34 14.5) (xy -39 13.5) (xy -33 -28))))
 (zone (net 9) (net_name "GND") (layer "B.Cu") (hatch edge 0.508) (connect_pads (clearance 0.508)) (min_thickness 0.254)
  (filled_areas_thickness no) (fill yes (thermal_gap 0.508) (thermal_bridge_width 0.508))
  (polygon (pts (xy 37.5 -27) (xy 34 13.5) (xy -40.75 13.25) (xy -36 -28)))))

